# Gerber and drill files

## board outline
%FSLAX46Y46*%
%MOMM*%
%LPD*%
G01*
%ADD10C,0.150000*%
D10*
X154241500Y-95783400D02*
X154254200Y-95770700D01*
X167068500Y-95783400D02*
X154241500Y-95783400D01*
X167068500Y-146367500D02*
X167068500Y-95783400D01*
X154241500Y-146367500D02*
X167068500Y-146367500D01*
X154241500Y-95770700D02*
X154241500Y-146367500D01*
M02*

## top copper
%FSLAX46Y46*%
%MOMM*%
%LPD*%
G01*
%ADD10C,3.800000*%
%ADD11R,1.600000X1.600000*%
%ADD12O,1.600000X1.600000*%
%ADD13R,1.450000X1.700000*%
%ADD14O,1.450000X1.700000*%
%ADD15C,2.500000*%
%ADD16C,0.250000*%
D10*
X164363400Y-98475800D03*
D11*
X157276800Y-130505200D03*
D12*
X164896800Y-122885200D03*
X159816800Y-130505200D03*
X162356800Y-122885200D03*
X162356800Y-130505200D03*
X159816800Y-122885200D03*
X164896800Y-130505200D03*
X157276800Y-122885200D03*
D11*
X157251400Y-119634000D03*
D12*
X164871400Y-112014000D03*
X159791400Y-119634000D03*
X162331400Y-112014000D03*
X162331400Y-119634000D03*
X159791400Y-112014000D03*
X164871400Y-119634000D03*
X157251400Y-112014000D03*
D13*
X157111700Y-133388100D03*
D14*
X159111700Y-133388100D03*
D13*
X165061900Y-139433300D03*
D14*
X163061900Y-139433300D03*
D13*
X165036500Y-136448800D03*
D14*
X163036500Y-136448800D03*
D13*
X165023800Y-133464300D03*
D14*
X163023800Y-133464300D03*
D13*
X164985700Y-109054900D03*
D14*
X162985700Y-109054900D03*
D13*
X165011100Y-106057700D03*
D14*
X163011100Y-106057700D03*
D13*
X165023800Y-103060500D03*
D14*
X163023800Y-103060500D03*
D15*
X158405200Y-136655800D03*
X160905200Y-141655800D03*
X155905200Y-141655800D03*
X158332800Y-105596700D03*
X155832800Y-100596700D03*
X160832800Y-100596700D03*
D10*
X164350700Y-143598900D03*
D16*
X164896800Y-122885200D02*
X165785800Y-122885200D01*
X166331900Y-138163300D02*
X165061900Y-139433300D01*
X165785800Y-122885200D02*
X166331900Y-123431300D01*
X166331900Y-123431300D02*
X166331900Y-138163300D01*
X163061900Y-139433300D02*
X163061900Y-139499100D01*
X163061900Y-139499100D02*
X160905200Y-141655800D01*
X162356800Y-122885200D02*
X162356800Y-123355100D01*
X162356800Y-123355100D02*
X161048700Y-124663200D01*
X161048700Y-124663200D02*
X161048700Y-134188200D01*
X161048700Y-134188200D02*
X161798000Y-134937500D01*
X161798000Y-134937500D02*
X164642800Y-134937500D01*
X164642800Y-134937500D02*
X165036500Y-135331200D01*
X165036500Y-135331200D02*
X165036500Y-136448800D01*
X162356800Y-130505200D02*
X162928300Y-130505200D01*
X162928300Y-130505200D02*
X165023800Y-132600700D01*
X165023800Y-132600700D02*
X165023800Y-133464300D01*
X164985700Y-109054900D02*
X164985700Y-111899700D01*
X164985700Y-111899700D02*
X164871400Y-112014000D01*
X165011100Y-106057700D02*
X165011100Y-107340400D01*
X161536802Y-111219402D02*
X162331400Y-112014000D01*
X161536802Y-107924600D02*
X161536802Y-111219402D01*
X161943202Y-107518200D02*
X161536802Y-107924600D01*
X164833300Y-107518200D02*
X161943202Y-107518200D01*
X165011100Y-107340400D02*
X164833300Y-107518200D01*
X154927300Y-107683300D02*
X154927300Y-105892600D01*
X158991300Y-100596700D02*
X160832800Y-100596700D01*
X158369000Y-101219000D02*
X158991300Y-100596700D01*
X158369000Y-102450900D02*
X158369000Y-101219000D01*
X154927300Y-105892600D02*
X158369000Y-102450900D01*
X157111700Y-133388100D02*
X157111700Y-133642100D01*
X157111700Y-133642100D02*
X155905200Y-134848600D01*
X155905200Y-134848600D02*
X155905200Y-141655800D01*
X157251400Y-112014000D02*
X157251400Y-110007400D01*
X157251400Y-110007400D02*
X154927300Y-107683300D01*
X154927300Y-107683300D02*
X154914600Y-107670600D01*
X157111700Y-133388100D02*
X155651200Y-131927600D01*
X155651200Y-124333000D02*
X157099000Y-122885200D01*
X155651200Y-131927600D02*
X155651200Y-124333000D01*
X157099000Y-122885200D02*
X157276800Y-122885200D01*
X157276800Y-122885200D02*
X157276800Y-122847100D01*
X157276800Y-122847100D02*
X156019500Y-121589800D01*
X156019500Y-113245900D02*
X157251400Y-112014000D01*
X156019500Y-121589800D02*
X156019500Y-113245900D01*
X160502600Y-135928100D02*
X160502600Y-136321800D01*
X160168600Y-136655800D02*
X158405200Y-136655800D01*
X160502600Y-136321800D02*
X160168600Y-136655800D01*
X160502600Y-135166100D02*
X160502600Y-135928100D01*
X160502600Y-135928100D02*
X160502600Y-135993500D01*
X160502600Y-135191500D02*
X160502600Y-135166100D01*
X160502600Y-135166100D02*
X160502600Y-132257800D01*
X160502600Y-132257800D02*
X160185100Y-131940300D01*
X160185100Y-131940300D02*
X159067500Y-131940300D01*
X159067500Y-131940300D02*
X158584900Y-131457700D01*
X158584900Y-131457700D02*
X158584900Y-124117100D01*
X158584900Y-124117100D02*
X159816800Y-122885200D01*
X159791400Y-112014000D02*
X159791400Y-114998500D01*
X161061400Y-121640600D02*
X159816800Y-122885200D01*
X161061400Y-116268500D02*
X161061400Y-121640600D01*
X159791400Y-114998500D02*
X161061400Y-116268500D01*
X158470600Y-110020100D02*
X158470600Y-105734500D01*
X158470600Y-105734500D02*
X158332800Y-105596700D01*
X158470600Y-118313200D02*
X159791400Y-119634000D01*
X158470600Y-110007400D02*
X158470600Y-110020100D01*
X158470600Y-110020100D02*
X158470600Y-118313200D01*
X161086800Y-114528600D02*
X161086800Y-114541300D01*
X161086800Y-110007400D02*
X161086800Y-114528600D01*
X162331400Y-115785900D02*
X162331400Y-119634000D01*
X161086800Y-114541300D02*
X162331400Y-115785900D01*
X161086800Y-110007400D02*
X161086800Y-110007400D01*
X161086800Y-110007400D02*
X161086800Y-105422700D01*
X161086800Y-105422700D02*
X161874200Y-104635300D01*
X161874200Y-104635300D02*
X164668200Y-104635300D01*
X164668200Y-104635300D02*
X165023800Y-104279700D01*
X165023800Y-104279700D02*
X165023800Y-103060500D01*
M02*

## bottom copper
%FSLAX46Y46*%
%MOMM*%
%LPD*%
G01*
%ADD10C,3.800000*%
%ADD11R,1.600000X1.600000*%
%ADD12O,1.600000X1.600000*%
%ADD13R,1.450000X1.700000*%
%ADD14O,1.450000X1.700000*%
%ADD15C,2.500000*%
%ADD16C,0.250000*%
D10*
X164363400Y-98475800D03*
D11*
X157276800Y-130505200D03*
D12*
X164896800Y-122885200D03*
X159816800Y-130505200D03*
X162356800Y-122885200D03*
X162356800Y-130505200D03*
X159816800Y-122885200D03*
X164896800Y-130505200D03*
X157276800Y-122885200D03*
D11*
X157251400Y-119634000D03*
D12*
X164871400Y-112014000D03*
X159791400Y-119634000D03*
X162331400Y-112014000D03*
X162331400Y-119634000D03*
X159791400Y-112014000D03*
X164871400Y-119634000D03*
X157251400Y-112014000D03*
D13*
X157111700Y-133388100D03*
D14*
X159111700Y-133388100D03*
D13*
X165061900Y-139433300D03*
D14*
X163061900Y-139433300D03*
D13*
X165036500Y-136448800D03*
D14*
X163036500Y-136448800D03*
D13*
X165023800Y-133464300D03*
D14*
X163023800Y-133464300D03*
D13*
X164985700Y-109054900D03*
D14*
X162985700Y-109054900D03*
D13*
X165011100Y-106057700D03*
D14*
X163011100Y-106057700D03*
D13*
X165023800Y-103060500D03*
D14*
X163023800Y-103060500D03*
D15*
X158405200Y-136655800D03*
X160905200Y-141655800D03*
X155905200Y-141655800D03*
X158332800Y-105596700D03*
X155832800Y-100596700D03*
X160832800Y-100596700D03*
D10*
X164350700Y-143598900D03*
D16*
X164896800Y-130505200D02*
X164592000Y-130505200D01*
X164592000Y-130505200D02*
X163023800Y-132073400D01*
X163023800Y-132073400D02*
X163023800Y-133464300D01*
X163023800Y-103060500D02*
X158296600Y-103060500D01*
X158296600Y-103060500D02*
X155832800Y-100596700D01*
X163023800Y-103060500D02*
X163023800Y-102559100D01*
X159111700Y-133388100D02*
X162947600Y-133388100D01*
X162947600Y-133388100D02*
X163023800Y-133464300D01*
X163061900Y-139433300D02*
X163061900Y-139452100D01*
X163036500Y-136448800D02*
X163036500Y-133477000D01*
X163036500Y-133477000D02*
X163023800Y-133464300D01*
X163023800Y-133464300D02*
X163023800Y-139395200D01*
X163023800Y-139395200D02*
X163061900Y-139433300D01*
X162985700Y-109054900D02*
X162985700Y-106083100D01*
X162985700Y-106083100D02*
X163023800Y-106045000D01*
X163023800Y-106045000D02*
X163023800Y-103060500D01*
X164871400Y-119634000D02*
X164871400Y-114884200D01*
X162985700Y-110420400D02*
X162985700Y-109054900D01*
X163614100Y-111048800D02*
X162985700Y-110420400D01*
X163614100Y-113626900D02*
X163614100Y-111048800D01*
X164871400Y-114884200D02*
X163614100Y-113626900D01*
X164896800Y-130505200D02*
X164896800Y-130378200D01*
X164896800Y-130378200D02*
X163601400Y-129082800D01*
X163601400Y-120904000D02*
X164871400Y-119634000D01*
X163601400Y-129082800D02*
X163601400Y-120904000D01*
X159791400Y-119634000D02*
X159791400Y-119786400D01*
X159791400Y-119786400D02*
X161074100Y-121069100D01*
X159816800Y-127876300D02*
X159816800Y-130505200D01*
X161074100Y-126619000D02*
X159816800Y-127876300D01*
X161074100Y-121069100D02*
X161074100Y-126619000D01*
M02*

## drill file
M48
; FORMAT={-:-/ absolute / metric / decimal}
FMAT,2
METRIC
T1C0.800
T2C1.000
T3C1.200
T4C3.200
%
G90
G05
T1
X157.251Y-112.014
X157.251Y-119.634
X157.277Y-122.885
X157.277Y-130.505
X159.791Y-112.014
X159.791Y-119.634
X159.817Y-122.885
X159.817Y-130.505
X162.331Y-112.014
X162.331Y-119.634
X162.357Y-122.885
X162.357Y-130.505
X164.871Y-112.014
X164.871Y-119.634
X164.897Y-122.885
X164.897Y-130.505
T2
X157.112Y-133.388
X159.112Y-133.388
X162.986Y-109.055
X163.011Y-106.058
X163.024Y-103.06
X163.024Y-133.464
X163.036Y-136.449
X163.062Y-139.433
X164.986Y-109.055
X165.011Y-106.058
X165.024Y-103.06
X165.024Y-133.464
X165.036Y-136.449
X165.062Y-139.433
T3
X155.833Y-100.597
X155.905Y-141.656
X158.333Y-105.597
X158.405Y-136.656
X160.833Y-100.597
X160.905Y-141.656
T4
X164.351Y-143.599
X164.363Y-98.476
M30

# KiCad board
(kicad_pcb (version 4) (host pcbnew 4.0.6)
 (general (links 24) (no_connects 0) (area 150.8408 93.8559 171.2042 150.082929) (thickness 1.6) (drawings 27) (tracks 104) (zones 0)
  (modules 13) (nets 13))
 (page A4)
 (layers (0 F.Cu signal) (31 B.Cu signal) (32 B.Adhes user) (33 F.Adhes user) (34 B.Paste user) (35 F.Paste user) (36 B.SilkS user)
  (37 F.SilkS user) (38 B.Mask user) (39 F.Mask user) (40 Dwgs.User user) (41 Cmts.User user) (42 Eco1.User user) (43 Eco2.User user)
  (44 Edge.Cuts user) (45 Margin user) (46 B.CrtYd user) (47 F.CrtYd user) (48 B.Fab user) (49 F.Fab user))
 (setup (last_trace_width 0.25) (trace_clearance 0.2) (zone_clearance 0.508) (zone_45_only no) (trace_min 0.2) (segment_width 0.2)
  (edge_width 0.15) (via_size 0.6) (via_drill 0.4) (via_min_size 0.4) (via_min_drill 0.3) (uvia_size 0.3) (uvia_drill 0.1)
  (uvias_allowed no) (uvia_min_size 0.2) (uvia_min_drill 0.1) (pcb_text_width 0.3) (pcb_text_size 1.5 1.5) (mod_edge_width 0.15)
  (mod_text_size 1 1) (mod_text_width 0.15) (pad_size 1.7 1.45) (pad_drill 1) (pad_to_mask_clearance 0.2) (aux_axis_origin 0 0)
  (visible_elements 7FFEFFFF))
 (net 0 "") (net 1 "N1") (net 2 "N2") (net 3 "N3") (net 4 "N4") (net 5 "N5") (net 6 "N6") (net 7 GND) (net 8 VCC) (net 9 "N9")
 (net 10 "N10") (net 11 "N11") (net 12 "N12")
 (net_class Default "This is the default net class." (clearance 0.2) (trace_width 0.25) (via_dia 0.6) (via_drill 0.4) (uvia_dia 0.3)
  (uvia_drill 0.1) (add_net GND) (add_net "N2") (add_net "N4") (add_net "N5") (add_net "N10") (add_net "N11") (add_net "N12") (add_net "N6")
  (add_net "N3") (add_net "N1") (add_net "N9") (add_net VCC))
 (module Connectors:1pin (layer F.Cu) (at 164.3634 98.4758)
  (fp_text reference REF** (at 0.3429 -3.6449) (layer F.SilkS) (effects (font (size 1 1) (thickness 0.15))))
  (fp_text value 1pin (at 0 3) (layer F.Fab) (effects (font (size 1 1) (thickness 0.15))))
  (pad 1 thru_hole circle (at 0 0) (size 3.8 3.8) (drill 3.2) (layers *.Cu *.Mask)))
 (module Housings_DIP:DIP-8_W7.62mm (layer F.Cu) (at 157.2768 130.5052 90)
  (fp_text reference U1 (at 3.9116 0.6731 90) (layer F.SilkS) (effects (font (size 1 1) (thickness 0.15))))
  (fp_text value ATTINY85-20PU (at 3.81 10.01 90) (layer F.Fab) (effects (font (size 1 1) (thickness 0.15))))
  (pad 1 thru_hole rect (at 0 0 90) (size 1.6 1.6) (drill 0.8) (layers *.Cu *.Mask) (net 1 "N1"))
  (pad 5 thru_hole oval (at 7.62 7.62 90) (size 1.6 1.6) (drill 0.8) (layers *.Cu *.Mask) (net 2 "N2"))
  (pad 2 thru_hole oval (at 0 2.54 90) (size 1.6 1.6) (drill 0.8) (layers *.Cu *.Mask) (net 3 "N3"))
  (pad 6 thru_hole oval (at 7.62 5.08 90) (size 1.6 1.6) (drill 0.8) (layers *.Cu *.Mask) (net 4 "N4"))
  (pad 3 thru_hole oval (at 0 5.08 90) (size 1.6 1.6) (drill 0.8) (layers *.Cu *.Mask) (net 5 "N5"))
  (pad 7 thru_hole oval (at 7.62 2.54 90) (size 1.6 1.6) (drill 0.8) (layers *.Cu *.Mask) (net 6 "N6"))
  (pad 4 thru_hole oval (at 0 7.62 90) (size 1.6 1.6) (drill 0.8) (layers *.Cu *.Mask) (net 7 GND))
  (pad 8 thru_hole oval (at 7.62 0 90) (size 1.6 1.6) (drill 0.8) (layers *.Cu *.Mask) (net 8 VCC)))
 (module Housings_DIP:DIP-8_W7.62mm (layer F.Cu) (at 157.2514 119.634 90)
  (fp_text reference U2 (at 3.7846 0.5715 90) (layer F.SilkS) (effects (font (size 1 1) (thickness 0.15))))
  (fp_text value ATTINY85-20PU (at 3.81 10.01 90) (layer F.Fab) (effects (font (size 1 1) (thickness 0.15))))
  (pad 1 thru_hole rect (at 0 0 90) (size 1.6 1.6) (drill 0.8) (layers *.Cu *.Mask) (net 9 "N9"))
  (pad 5 thru_hole oval (at 7.62 7.62 90) (size 1.6 1.6) (drill 0.8) (layers *.Cu *.Mask) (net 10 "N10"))
  (pad 2 thru_hole oval (at 0 2.54 90) (size 1.6 1.6) (drill 0.8) (layers *.Cu *.Mask) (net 3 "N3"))
  (pad 6 thru_hole oval (at 7.62 5.08 90) (size 1.6 1.6) (drill 0.8) (layers *.Cu *.Mask) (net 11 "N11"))
  (pad 3 thru_hole oval (at 0 5.08 90) (size 1.6 1.6) (drill 0.8) (layers *.Cu *.Mask) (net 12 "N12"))
  (pad 7 thru_hole oval (at 7.62 2.54 90) (size 1.6 1.6) (drill 0.8) (layers *.Cu *.Mask) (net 6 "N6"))
  (pad 4 thru_hole oval (at 0 7.62 90) (size 1.6 1.6) (drill 0.8) (layers *.Cu *.Mask) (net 7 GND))
  (pad 8 thru_hole oval (at 7.62 0 90) (size 1.6 1.6) (drill 0.8) (layers *.Cu *.Mask) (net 8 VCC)))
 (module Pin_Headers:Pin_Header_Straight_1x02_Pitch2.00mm (layer F.Cu) (at 157.1117 133.3881 90)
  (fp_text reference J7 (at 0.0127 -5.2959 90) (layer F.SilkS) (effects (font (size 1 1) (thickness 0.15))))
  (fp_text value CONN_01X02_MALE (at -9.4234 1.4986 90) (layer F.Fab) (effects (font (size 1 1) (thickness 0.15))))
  (pad 1 thru_hole rect (at 0 0 90) (size 1.7 1.45) (drill 1) (layers *.Cu *.Mask) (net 8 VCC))
  (pad 2 thru_hole oval (at 0 2 90) (size 1.7 1.45) (drill 1) (layers *.Cu *.Mask) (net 7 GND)))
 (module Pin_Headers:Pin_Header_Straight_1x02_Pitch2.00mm (layer F.Cu) (at 165.0619 139.4333 270)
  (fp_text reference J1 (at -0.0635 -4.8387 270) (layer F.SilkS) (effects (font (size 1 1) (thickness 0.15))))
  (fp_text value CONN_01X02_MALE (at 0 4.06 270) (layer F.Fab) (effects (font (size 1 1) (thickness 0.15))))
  (pad 1 thru_hole rect (at 0 0 270) (size 1.7 1.45) (drill 1) (layers *.Cu *.Mask) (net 2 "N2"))
  (pad 2 thru_hole oval (at 0 2 270) (size 1.7 1.45) (drill 1) (layers *.Cu *.Mask) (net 7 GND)))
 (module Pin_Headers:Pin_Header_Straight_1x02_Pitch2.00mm (layer F.Cu) (at 165.0365 136.4488 270)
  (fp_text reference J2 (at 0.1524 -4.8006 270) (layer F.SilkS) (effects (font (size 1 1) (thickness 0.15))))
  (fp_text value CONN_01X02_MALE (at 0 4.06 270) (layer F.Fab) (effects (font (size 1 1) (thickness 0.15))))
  (pad 1 thru_hole rect (at 0 0 270) (size 1.7 1.45) (drill 1) (layers *.Cu *.Mask) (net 4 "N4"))
  (pad 2 thru_hole oval (at 0 2 270) (size 1.7 1.45) (drill 1) (layers *.Cu *.Mask) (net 7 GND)))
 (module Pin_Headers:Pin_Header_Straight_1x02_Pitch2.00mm (layer F.Cu) (at 165.0238 133.4643 270)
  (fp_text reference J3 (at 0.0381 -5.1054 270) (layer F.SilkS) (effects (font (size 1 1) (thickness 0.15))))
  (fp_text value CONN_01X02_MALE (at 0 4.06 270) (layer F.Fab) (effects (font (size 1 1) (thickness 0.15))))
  (pad 1 thru_hole rect (at 0 0 270) (size 1.7 1.45) (drill 1) (layers *.Cu *.Mask) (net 5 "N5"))
  (pad 2 thru_hole oval (at 0 2 270) (size 1.7 1.45) (drill 1) (layers *.Cu *.Mask) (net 7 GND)))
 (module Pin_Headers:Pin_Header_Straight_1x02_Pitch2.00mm (layer F.Cu) (at 164.9857 109.0549 270)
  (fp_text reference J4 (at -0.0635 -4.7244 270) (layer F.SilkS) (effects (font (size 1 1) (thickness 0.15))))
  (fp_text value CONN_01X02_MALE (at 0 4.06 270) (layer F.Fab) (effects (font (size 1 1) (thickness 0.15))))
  (pad 1 thru_hole rect (at 0 0 270) (size 1.7 1.45) (drill 1) (layers *.Cu *.Mask) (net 10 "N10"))
  (pad 2 thru_hole oval (at 0 2 270) (size 1.7 1.45) (drill 1) (layers *.Cu *.Mask) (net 7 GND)))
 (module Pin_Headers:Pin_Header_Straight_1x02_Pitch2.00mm (layer F.Cu) (at 165.0111 106.0577 270)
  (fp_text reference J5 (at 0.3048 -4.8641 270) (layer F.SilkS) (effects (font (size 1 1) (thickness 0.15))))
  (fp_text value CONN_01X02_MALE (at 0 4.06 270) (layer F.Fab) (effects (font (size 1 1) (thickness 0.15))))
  (pad 1 thru_hole rect (at 0 0 270) (size 1.7 1.45) (drill 1) (layers *.Cu *.Mask) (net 11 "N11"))
  (pad 2 thru_hole oval (at 0 2 270) (size 1.7 1.45) (drill 1) (layers *.Cu *.Mask) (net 7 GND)))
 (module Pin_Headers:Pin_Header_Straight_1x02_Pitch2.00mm (layer F.Cu) (at 165.0238 103.0605 270)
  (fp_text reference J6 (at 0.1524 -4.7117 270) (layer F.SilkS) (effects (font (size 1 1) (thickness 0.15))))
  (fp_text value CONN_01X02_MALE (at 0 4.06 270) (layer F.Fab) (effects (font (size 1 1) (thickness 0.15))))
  (pad 1 thru_hole rect (at 0 0 270) (size 1.7 1.45) (drill 1) (layers *.Cu *.Mask) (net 12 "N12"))
  (pad 2 thru_hole oval (at 0 2 270) (size 1.7 1.45) (drill 1) (layers *.Cu *.Mask) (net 7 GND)))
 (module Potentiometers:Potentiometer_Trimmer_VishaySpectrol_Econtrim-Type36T (layer F.Cu) (at 155.9052 141.6558)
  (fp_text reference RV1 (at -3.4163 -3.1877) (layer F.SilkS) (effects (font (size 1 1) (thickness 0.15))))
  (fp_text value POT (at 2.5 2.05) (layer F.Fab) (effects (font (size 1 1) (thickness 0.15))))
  (pad 2 thru_hole circle (at 2.5 -5) (size 2.5 2.5) (drill 1.2) (layers *.Cu *.Mask) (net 6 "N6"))
  (pad 3 thru_hole circle (at 5 0) (size 2.5 2.5) (drill 1.2) (layers *.Cu *.Mask) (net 7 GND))
  (pad 1 thru_hole circle (at 0 0) (size 2.5 2.5) (drill 1.2) (layers *.Cu *.Mask) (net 8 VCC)))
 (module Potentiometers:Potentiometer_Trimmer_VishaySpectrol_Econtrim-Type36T (layer F.Cu) (at 160.8328 100.5967 180)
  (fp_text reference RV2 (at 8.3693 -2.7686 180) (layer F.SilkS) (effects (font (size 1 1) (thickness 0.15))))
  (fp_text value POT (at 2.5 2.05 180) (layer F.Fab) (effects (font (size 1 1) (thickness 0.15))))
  (pad 2 thru_hole circle (at 2.5 -5 180) (size 2.5 2.5) (drill 1.2) (layers *.Cu *.Mask) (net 3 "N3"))
  (pad 3 thru_hole circle (at 5 0 180) (size 2.5 2.5) (drill 1.2) (layers *.Cu *.Mask) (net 7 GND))
  (pad 1 thru_hole circle (at 0 0 180) (size 2.5 2.5) (drill 1.2) (layers *.Cu *.Mask) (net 8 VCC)))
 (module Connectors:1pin (layer F.Cu) (at 164.3507 143.5989)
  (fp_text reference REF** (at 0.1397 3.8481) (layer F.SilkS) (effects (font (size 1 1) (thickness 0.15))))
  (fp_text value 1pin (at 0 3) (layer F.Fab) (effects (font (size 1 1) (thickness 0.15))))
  (pad 1 thru_hole circle (at 0 0) (size 3.8 3.8) (drill 3.2) (layers *.Cu *.Mask)))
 (gr_line (start 154.2415 95.7834) (end 154.2542 95.7707) (angle 90) (layer Edge.Cuts) (width 0.15))
 (gr_line (start 167.0685 95.7834) (end 154.2415 95.7834) (angle 90) (layer Edge.Cuts) (width 0.15))
 (gr_line (start 167.0685 146.3675) (end 167.0685 95.7834) (angle 90) (layer Edge.Cuts) (width 0.15))
 (gr_line (start 154.2415 146.3675) (end 167.0685 146.3675) (angle 90) (layer Edge.Cuts) (width 0.15))
 (gr_line (start 154.2415 95.7707) (end 154.2415 146.3675) (angle 90) (layer Edge.Cuts) (width 0.15))
 (segment (start 164.8968 122.8852) (end 165.7858 122.8852) (width 0.25) (layer F.Cu) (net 2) (status 10))
 (segment (start 166.3319 138.1633) (end 165.0619 139.4333) (width 0.25) (layer F.Cu) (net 2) (status 20))
 (segment (start 165.7858 122.8852) (end 166.3319 123.4313) (width 0.25) (layer F.Cu) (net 2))
 (segment (start 166.3319 123.4313) (end 166.3319 138.1633) (width 0.25) (layer F.Cu) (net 2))
 (segment (start 164.8968 130.5052) (end 164.592 130.5052) (width 0.25) (layer B.Cu) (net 7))
 (segment (start 164.592 130.5052) (end 163.0238 132.0734) (width 0.25) (layer B.Cu) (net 7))
 (segment (start 163.0238 132.0734) (end 163.0238 133.4643) (width 0.25) (layer B.Cu) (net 7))
 (segment (start 163.0238 103.0605) (end 158.2966 103.0605) (width 0.25) (layer B.Cu) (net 7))
 (segment (start 158.2966 103.0605) (end 155.8328 100.5967) (width 0.25) (layer B.Cu) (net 7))
 (segment (start 163.0619 139.4333) (end 163.0619 139.4991) (width 0.25) (layer F.Cu) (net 7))
 (segment (start 163.0619 139.4991) (end 160.9052 141.6558) (width 0.25) (layer F.Cu) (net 7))
 (segment (start 163.0238 103.0605) (end 163.0238 102.5591) (width 0.25) (layer B.Cu) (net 7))
 (segment (start 159.1117 133.3881) (end 162.9476 133.3881) (width 0.25) (layer B.Cu) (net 7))
 (segment (start 162.9476 133.3881) (end 163.0238 133.4643) (width 0.25) (layer B.Cu) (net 7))
 (segment (start 163.0619 139.4333) (end 163.0619 139.4521) (width 0.25) (layer B.Cu) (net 7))
 (segment (start 163.0365 136.4488) (end 163.0365 133.477) (width 0.25) (layer B.Cu) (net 7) (status 30))
 (segment (start 163.0365 133.477) (end 163.0238 133.4643) (width 0.25) (layer B.Cu) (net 7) (status 30))
 (segment (start 163.0238 133.4643) (end 163.0238 139.3952) (width 0.25) (layer B.Cu) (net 7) (status 30))
 (segment (start 163.0238 139.3952) (end 163.0619 139.4333) (width 0.25) (layer B.Cu) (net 7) (status 30))
 (segment (start 162.9857 109.0549) (end 162.9857 106.0831) (width 0.25) (layer B.Cu) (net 7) (status 30))
 (segment (start 162.9857 106.0831) (end 163.0238 106.045) (width 0.25) (layer B.Cu) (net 7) (status 30))
 (segment (start 163.0238 106.045) (end 163.0238 103.0605) (width 0.25) (layer B.Cu) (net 7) (status 30))
 (segment (start 164.8714 119.634) (end 164.8714 114.8842) (width 0.25) (layer B.Cu) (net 7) (status 10))
 (segment (start 162.9857 110.4204) (end 162.9857 109.0549) (width 0.25) (layer B.Cu) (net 7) (status 20))
 (segment (start 163.6141 111.0488) (end 162.9857 110.4204) (width 0.25) (layer B.Cu) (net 7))
 (segment (start 163.6141 113.6269) (end 163.6141 111.0488) (width 0.25) (layer B.Cu) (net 7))
 (segment (start 164.8714 114.8842) (end 163.6141 113.6269) (width 0.25) (layer B.Cu) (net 7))
 (segment (start 164.8968 130.5052) (end 164.8968 130.3782) (width 0.25) (layer B.Cu) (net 7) (status 30))
 (segment (start 164.8968 130.3782) (end 163.6014 129.0828) (width 0.25) (layer B.Cu) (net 7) (status 10))
 (segment (start 163.6014 120.904) (end 164.8714 119.634) (width 0.25) (layer B.Cu) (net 7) (status 20))
 (segment (start 163.6014 129.0828) (end 163.6014 120.904) (width 0.25) (layer B.Cu) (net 7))
 (segment (start 162.3568 122.8852) (end 162.3568 123.3551) (width 0.25) (layer F.Cu) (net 4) (status 30))
 (segment (start 162.3568 123.3551) (end 161.0487 124.6632) (width 0.25) (layer F.Cu) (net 4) (status 10))
 (segment (start 161.0487 124.6632) (end 161.0487 134.1882) (width 0.25) (layer F.Cu) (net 4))
 (segment (start 161.0487 134.1882) (end 161.798 134.9375) (width 0.25) (layer F.Cu) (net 4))
 (segment (start 161.798 134.9375) (end 164.6428 134.9375) (width 0.25) (layer F.Cu) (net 4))
 (segment (start 164.6428 134.9375) (end 165.0365 135.3312) (width 0.25) (layer F.Cu) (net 4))
 (segment (start 165.0365 135.3312) (end 165.0365 136.4488) (width 0.25) (layer F.Cu) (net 4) (status 20))
 (segment (start 162.3568 130.5052) (end 162.9283 130.5052) (width 0.25) (layer F.Cu) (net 5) (status 30))
 (segment (start 162.9283 130.5052) (end 165.0238 132.6007) (width 0.25) (layer F.Cu) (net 5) (status 10))
 (segment (start 165.0238 132.6007) (end 165.0238 133.4643) (width 0.25) (layer F.Cu) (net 5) (status 20))
 (segment (start 164.9857 109.0549) (end 164.9857 111.8997) (width 0.25) (layer F.Cu) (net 10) (status 30))
 (segment (start 164.9857 111.8997) (end 164.8714 112.014) (width 0.25) (layer F.Cu) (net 10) (status 30))
 (segment (start 165.0111 106.0577) (end 165.0111 107.3404) (width 0.25) (layer F.Cu) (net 11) (status 10))
 (segment (start 161.536802 111.219402) (end 162.3314 112.014) (width 0.25) (layer F.Cu) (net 11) (status 20))
 (segment (start 161.536802 107.9246) (end 161.536802 111.219402) (width 0.25) (layer F.Cu) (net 11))
 (segment (start 161.943202 107.5182) (end 161.536802 107.9246) (width 0.25) (layer F.Cu) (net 11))
 (segment (start 164.8333 107.5182) (end 161.943202 107.5182) (width 0.25) (layer F.Cu) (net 11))
 (segment (start 165.0111 107.3404) (end 164.8333 107.5182) (width 0.25) (layer F.Cu) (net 11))
 (segment (start 154.9273 107.6833) (end 154.9273 105.8926) (width 0.25) (layer F.Cu) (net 8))
 (segment (start 158.9913 100.5967) (end 160.8328 100.5967) (width 0.25) (layer F.Cu) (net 8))
 (segment (start 158.369 101.219) (end 158.9913 100.5967) (width 0.25) (layer F.Cu) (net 8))
 (segment (start 158.369 102.4509) (end 158.369 101.219) (width 0.25) (layer F.Cu) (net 8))
 (segment (start 154.9273 105.8926) (end 158.369 102.4509) (width 0.25) (layer F.Cu) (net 8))
 (segment (start 157.1117 133.3881) (end 157.1117 133.6421) (width 0.25) (layer F.Cu) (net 8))
 (segment (start 157.1117 133.6421) (end 155.9052 134.8486) (width 0.25) (layer F.Cu) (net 8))
 (segment (start 155.9052 134.8486) (end 155.9052 141.6558) (width 0.25) (layer F.Cu) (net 8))
 (segment (start 157.2514 112.014) (end 157.2514 110.0074) (width 0.25) (layer F.Cu) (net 8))
 (segment (start 157.2514 110.0074) (end 154.9273 107.6833) (width 0.25) (layer F.Cu) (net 8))
 (segment (start 154.9273 107.6833) (end 154.9146 107.6706) (width 0.25) (layer F.Cu) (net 8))
 (segment (start 157.1117 133.3881) (end 155.6512 131.9276) (width 0.25) (layer F.Cu) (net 8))
 (segment (start 155.6512 124.333) (end 157.099 122.8852) (width 0.25) (layer F.Cu) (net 8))
 (segment (start 155.6512 131.9276) (end 155.6512 124.333) (width 0.25) (layer F.Cu) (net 8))
 (segment (start 157.099 122.8852) (end 157.2768 122.8852) (width 0.25) (layer F.Cu) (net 8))
 (segment (start 157.2768 122.8852) (end 157.2768 122.8471) (width 0.25) (layer F.Cu) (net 8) (status 30))
 (segment (start 157.2768 122.8471) (end 156.0195 121.5898) (width 0.25) (layer F.Cu) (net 8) (status 10))
 (segment (start 156.0195 113.2459) (end 157.2514 112.014) (width 0.25) (layer F.Cu) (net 8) (status 20))
 (segment (start 156.0195 121.5898) (end 156.0195 113.2459) (width 0.25) (layer F.Cu) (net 8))
 (segment (start 160.5026 135.9281) (end 160.5026 136.3218) (width 0.25) (layer F.Cu) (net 6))
 (segment (start 160.1686 136.6558) (end 158.4052 136.6558) (width 0.25) (layer F.Cu) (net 6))
 (segment (start 160.5026 136.3218) (end 160.1686 136.6558) (width 0.25) (layer F.Cu) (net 6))
 (segment (start 160.5026 135.1661) (end 160.5026 135.9281) (width 0.25) (layer F.Cu) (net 6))
 (segment (start 160.5026 135.9281) (end 160.5026 135.9935) (width 0.25) (layer F.Cu) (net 6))
 (segment (start 160.5026 135.1915) (end 160.5026 135.1661) (width 0.25) (layer F.Cu) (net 6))
 (segment (start 160.5026 135.1661) (end 160.5026 132.2578) (width 0.25) (layer F.Cu) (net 6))
 (segment (start 160.5026 132.2578) (end 160.1851 131.9403) (width 0.25) (layer F.Cu) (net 6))
 (segment (start 160.1851 131.9403) (end 159.0675 131.9403) (width 0.25) (layer F.Cu) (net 6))
 (segment (start 159.0675 131.9403) (end 158.5849 131.4577) (width 0.25) (layer F.Cu) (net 6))
 (segment (start 158.5849 131.4577) (end 158.5849 124.1171) (width 0.25) (layer F.Cu) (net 6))
 (segment (start 158.5849 124.1171) (end 159.8168 122.8852) (width 0.25) (layer F.Cu) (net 6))
 (segment (start 159.7914 112.014) (end 159.7914 114.9985) (width 0.25) (layer F.Cu) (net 6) (status 10))
 (segment (start 161.0614 121.6406) (end 159.8168 122.8852) (width 0.25) (layer F.Cu) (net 6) (status 20))
 (segment (start 161.0614 116.2685) (end 161.0614 121.6406) (width 0.25) (layer F.Cu) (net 6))
 (segment (start 159.7914 114.9985) (end 161.0614 116.2685) (width 0.25) (layer F.Cu) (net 6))
 (segment (start 158.4706 110.0201) (end 158.4706 105.7345) (width 0.25) (layer F.Cu) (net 3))
 (segment (start 158.4706 105.7345) (end 158.3328 105.5967) (width 0.25) (layer F.Cu) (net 3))
 (segment (start 158.4706 118.3132) (end 159.7914 119.634) (width 0.25) (layer F.Cu) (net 3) (status 20))
 (segment (start 158.4706 110.0074) (end 158.4706 110.0201) (width 0.25) (layer F.Cu) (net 3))
 (segment (start 158.4706 110.0201) (end 158.4706 118.3132) (width 0.25) (layer F.Cu) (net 3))
 (segment (start 159.7914 119.634) (end 159.7914 119.7864) (width 0.25) (layer B.Cu) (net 3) (status 30))
 (segment (start 159.7914 119.7864) (end 161.0741 121.0691) (width 0.25) (layer B.Cu) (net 3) (status 10))
 (segment (start 159.8168 127.8763) (end 159.8168 130.5052) (width 0.25) (layer B.Cu) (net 3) (status 20))
 (segment (start 161.0741 126.619) (end 159.8168 127.8763) (width 0.25) (layer B.Cu) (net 3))
 (segment (start 161.0741 121.0691) (end 161.0741 126.619) (width 0.25) (layer B.Cu) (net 3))
 (segment (start 161.0868 114.5286) (end 161.0868 114.5413) (width 0.25) (layer F.Cu) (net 12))
 (segment (start 161.0868 110.0074) (end 161.0868 114.5286) (width 0.25) (layer F.Cu) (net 12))
 (segment (start 162.3314 115.7859) (end 162.3314 119.634) (width 0.25) (layer F.Cu) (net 12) (status 20))
 (segment (start 161.0868 114.5413) (end 162.3314 115.7859) (width 0.25) (layer F.Cu) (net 12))
 (segment (start 161.0868 110.0074) (end 161.0868 110.0074) (width 0.25) (layer F.Cu) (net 12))
 (segment (start 161.0868 110.0074) (end 161.0868 105.4227) (width 0.25) (layer F.Cu) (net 12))
 (segment (start 161.0868 105.4227) (end 161.8742 104.6353) (width 0.25) (layer F.Cu) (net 12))
 (segment (start 161.8742 104.6353) (end 164.6682 104.6353) (width 0.25) (layer F.Cu) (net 12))
 (segment (start 164.6682 104.6353) (end 165.0238 104.2797) (width 0.25) (layer F.Cu) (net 12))
 (segment (start 165.0238 104.2797) (end 165.0238 103.0605) (width 0.25) (layer F.Cu) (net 12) (status 20)))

